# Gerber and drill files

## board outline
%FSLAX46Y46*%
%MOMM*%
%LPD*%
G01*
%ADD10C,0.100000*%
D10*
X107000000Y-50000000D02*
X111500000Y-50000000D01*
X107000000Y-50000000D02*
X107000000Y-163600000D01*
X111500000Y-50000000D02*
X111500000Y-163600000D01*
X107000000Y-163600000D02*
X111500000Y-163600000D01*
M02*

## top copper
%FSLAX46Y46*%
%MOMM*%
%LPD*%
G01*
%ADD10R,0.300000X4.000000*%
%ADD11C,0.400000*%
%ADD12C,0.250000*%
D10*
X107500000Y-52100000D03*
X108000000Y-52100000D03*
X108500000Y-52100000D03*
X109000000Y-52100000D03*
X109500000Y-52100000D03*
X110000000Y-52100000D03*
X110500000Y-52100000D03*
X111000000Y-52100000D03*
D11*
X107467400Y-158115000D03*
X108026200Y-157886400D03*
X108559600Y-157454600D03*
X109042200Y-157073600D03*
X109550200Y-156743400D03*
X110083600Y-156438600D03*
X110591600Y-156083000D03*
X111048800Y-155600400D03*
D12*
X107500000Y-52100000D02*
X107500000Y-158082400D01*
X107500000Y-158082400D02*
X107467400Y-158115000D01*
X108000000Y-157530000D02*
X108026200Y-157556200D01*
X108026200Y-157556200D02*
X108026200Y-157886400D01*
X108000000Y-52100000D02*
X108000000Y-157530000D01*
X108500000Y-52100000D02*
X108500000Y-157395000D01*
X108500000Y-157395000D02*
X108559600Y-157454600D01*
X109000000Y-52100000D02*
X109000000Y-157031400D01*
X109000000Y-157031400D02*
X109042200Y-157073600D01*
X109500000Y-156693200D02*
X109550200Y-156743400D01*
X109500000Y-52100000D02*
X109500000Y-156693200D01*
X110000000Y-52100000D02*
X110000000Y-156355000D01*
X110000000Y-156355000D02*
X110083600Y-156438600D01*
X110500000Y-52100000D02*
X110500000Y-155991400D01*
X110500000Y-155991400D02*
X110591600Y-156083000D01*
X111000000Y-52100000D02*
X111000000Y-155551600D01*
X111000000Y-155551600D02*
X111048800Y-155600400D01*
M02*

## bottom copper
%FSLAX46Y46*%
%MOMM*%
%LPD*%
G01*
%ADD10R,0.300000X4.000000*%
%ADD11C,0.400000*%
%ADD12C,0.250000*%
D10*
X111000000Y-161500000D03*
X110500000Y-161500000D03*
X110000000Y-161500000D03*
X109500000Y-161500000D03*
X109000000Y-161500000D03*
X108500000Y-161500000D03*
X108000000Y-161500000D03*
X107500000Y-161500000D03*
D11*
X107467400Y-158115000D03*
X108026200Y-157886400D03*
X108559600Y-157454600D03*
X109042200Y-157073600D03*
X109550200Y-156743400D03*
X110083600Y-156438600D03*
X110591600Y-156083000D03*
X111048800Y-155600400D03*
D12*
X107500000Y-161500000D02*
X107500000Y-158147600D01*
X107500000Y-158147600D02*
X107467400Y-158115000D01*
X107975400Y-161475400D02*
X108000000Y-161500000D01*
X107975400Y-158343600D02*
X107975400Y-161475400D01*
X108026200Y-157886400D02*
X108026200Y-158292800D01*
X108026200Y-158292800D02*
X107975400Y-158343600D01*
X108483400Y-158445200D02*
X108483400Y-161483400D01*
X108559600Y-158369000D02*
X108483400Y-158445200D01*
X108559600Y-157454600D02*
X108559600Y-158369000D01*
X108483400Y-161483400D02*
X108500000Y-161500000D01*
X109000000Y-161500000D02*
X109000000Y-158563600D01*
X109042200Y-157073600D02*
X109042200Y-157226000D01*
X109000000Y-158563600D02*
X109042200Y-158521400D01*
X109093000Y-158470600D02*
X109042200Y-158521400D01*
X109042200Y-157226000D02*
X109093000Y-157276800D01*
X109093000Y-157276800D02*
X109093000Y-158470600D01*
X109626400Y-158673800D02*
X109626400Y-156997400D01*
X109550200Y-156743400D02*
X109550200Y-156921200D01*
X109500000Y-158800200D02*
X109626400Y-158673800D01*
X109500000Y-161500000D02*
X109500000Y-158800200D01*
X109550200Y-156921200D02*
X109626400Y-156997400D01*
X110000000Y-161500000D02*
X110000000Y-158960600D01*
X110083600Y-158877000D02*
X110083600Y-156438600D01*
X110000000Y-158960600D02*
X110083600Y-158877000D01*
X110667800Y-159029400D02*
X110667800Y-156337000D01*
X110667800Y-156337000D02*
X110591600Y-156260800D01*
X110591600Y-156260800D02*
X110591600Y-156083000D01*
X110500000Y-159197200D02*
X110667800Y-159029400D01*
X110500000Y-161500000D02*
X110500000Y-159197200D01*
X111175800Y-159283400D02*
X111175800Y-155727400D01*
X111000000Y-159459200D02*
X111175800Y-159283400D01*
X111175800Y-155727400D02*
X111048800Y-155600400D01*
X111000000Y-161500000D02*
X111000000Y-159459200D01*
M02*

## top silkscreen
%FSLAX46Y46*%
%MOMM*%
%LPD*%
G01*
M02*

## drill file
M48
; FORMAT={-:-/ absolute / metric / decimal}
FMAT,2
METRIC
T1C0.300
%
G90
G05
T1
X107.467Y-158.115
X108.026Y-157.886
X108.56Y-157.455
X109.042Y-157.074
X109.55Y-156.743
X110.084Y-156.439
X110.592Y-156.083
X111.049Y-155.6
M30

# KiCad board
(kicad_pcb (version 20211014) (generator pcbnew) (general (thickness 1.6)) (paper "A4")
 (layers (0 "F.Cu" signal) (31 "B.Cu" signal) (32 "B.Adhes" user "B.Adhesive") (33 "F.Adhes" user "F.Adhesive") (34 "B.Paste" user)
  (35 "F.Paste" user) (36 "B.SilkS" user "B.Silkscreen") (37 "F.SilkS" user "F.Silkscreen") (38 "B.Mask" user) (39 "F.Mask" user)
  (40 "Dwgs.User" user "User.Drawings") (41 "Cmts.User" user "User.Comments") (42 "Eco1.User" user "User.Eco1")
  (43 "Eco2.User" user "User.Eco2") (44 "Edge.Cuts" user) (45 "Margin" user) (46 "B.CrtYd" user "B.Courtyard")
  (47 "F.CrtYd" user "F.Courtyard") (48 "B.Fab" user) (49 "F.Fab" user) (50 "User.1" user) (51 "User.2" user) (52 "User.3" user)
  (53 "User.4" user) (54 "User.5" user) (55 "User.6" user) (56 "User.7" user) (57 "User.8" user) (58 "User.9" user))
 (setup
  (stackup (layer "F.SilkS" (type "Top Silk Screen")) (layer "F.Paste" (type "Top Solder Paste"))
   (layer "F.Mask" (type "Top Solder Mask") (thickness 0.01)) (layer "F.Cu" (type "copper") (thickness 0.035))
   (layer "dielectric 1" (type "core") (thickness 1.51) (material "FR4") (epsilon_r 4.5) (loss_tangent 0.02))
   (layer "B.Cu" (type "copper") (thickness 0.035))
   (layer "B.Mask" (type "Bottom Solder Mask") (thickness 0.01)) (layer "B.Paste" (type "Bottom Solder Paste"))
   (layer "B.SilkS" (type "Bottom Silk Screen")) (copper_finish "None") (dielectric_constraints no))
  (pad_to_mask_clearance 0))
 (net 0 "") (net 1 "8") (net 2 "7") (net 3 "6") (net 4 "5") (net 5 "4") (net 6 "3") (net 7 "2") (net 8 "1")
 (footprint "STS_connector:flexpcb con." (layer "F.Cu") (at 107 54.1)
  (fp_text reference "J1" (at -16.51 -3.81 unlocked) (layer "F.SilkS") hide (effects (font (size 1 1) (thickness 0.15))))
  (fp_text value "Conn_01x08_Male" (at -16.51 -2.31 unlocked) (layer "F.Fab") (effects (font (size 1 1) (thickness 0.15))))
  (pad "1" smd rect (at 0.5 -2) (size 0.3 4) (layers "F.Cu" "F.Paste" "F.Mask") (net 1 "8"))
  (pad "2" smd rect (at 1 -2) (size 0.3 4) (layers "F.Cu" "F.Paste" "F.Mask") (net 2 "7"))
  (pad "3" smd rect (at 1.5 -2) (size 0.3 4) (layers "F.Cu" "F.Paste" "F.Mask") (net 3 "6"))
  (pad "4" smd rect (at 2 -2) (size 0.3 4) (layers "F.Cu" "F.Paste" "F.Mask") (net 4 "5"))
  (pad "5" smd rect (at 2.5 -2) (size 0.3 4) (layers "F.Cu" "F.Paste" "F.Mask") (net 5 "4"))
  (pad "6" smd rect (at 3 -2) (size 0.3 4) (layers "F.Cu" "F.Paste" "F.Mask") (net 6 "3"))
  (pad "7" smd rect (at 3.5 -2) (size 0.3 4) (layers "F.Cu" "F.Paste" "F.Mask") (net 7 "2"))
  (pad "8" smd rect (at 4 -2) (size 0.3 4) (layers "F.Cu" "F.Paste" "F.Mask") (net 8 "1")))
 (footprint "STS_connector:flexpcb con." (layer "B.Cu") (at 111.5 163.5 180)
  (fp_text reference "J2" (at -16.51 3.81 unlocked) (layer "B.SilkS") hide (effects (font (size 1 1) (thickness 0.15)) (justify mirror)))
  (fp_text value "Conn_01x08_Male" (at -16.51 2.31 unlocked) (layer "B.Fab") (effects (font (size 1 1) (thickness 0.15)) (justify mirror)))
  (pad "1" smd rect (at 0.5 2 180) (size 0.3 4) (layers "B.Cu" "B.Paste" "B.Mask") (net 8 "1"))
  (pad "2" smd rect (at 1 2 180) (size 0.3 4) (layers "B.Cu" "B.Paste" "B.Mask") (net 7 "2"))
  (pad "3" smd rect (at 1.5 2 180) (size 0.3 4) (layers "B.Cu" "B.Paste" "B.Mask") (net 6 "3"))
  (pad "4" smd rect (at 2 2 180) (size 0.3 4) (layers "B.Cu" "B.Paste" "B.Mask") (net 5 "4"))
  (pad "5" smd rect (at 2.5 2 180) (size 0.3 4) (layers "B.Cu" "B.Paste" "B.Mask") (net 4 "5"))
  (pad "6" smd rect (at 3 2 180) (size 0.3 4) (layers "B.Cu" "B.Paste" "B.Mask") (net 3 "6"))
  (pad "7" smd rect (at 3.5 2 180) (size 0.3 4) (layers "B.Cu" "B.Paste" "B.Mask") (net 2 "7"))
  (pad "8" smd rect (at 4 2 180) (size 0.3 4) (layers "B.Cu" "B.Paste" "B.Mask") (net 1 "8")))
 (gr_line (start 107 50) (end 111.5 50) (layer "Edge.Cuts") (width 0.1))
 (gr_line (start 107 50) (end 107 163.6) (layer "Edge.Cuts") (width 0.1))
 (gr_line (start 111.5 50) (end 111.5 163.6) (layer "Edge.Cuts") (width 0.1))
 (gr_line (start 107 163.6) (end 111.5 163.6) (layer "Edge.Cuts") (width 0.1))
 (segment (start 107.5 52.1) (end 107.5 158.0824) (width 0.25) (layer "F.Cu") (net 1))
 (segment (start 107.5 158.0824) (end 107.4674 158.115) (width 0.25) (layer "F.Cu") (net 1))
 (via (at 107.4674 158.115) (size 0.4) (drill 0.3) (layers "F.Cu" "B.Cu") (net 1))
 (segment (start 107.5 161.5) (end 107.5 158.1476) (width 0.25) (layer "B.Cu") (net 1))
 (segment (start 107.5 158.1476) (end 107.4674 158.115) (width 0.25) (layer "B.Cu") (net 1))
 (segment (start 108 157.53) (end 108.0262 157.5562) (width 0.25) (layer "F.Cu") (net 2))
 (segment (start 108.0262 157.5562) (end 108.0262 157.8864) (width 0.25) (layer "F.Cu") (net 2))
 (segment (start 108 52.1) (end 108 157.53) (width 0.25) (layer "F.Cu") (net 2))
 (via (at 108.0262 157.8864) (size 0.4) (drill 0.3) (layers "F.Cu" "B.Cu") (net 2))
 (segment (start 107.9754 161.4754) (end 108 161.5) (width 0.25) (layer "B.Cu") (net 2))
 (segment (start 107.9754 158.3436) (end 107.9754 161.4754) (width 0.25) (layer "B.Cu") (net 2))
 (segment (start 108.0262 157.8864) (end 108.0262 158.2928) (width 0.25) (layer "B.Cu") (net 2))
 (segment (start 108.0262 158.2928) (end 107.9754 158.3436) (width 0.25) (layer "B.Cu") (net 2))
 (segment (start 108.5 52.1) (end 108.5 157.395) (width 0.25) (layer "F.Cu") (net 3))
 (segment (start 108.5 157.395) (end 108.5596 157.4546) (width 0.25) (layer "F.Cu") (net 3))
 (via (at 108.5596 157.4546) (size 0.4) (drill 0.3) (layers "F.Cu" "B.Cu") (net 3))
 (segment (start 108.4834 158.4452) (end 108.4834 161.4834) (width 0.25) (layer "B.Cu") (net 3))
 (segment (start 108.5596 158.369) (end 108.4834 158.4452) (width 0.25) (layer "B.Cu") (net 3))
 (segment (start 108.5596 157.4546) (end 108.5596 158.369) (width 0.25) (layer "B.Cu") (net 3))
 (segment (start 108.4834 161.4834) (end 108.5 161.5) (width 0.25) (layer "B.Cu") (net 3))
 (segment (start 109 52.1) (end 109 157.0314) (width 0.25) (layer "F.Cu") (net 4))
 (segment (start 109 157.0314) (end 109.0422 157.0736) (width 0.25) (layer "F.Cu") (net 4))
 (via (at 109.0422 157.0736) (size 0.4) (drill 0.3) (layers "F.Cu" "B.Cu") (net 4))
 (segment (start 109 161.5) (end 109 158.5636) (width 0.25) (layer "B.Cu") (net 4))
 (segment (start 109.0422 157.0736) (end 109.0422 157.226) (width 0.25) (layer "B.Cu") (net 4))
 (segment (start 109 158.5636) (end 109.0422 158.5214) (width 0.25) (layer "B.Cu") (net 4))
 (segment (start 109.093 158.4706) (end 109.0422 158.5214) (width 0.25) (layer "B.Cu") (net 4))
 (segment (start 109.0422 157.226) (end 109.093 157.2768) (width 0.25) (layer "B.Cu") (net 4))
 (segment (start 109.093 157.2768) (end 109.093 158.4706) (width 0.25) (layer "B.Cu") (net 4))
 (segment (start 109.5 156.6932) (end 109.5502 156.7434) (width 0.25) (layer "F.Cu") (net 5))
 (segment (start 109.5 52.1) (end 109.5 156.6932) (width 0.25) (layer "F.Cu") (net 5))
 (via (at 109.5502 156.7434) (size 0.4) (drill 0.3) (layers "F.Cu" "B.Cu") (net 5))
 (segment (start 109.6264 158.6738) (end 109.6264 156.9974) (width 0.25) (layer "B.Cu") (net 5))
 (segment (start 109.5502 156.7434) (end 109.5502 156.9212) (width 0.25) (layer "B.Cu") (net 5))
 (segment (start 109.5 158.8002) (end 109.6264 158.6738) (width 0.25) (layer "B.Cu") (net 5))
 (segment (start 109.5 161.5) (end 109.5 158.8002) (width 0.25) (layer "B.Cu") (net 5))
 (segment (start 109.5502 156.9212) (end 109.6264 156.9974) (width 0.25) (layer "B.Cu") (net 5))
 (segment (start 110 52.1) (end 110 156.355) (width 0.25) (layer "F.Cu") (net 6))
 (segment (start 110 156.355) (end 110.0836 156.4386) (width 0.25) (layer "F.Cu") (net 6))
 (via (at 110.0836 156.4386) (size 0.4) (drill 0.3) (layers "F.Cu" "B.Cu") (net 6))
 (segment (start 110 161.5) (end 110 158.9606) (width 0.25) (layer "B.Cu") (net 6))
 (segment (start 110.0836 158.877) (end 110.0836 156.4386) (width 0.25) (layer "B.Cu") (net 6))
 (segment (start 110 158.9606) (end 110.0836 158.877) (width 0.25) (layer "B.Cu") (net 6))
 (segment (start 110.5 52.1) (end 110.5 155.9914) (width 0.25) (layer "F.Cu") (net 7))
 (segment (start 110.5 155.9914) (end 110.5916 156.083) (width 0.25) (layer "F.Cu") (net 7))
 (via (at 110.5916 156.083) (size 0.4) (drill 0.3) (layers "F.Cu" "B.Cu") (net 7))
 (segment (start 110.6678 159.0294) (end 110.6678 156.337) (width 0.25) (layer "B.Cu") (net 7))
 (segment (start 110.6678 156.337) (end 110.5916 156.2608) (width 0.25) (layer "B.Cu") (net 7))
 (segment (start 110.5916 156.2608) (end 110.5916 156.083) (width 0.25) (layer "B.Cu") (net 7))
 (segment (start 110.5 159.1972) (end 110.6678 159.0294) (width 0.25) (layer "B.Cu") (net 7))
 (segment (start 110.5 161.5) (end 110.5 159.1972) (width 0.25) (layer "B.Cu") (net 7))
 (segment (start 111 52.1) (end 111 155.5516) (width 0.25) (layer "F.Cu") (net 8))
 (segment (start 111 155.5516) (end 111.0488 155.6004) (width 0.25) (layer "F.Cu") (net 8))
 (via (at 111.0488 155.6004) (size 0.4) (drill 0.3) (layers "F.Cu" "B.Cu") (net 8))
 (segment (start 111.1758 159.2834) (end 111.1758 155.7274) (width 0.25) (layer "B.Cu") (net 8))
 (segment (start 111 159.4592) (end 111.1758 159.2834) (width 0.25) (layer "B.Cu") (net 8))
 (segment (start 111.1758 155.7274) (end 111.0488 155.6004) (width 0.25) (layer "B.Cu") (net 8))
 (segment (start 111 161.5) (end 111 159.4592) (width 0.25) (layer "B.Cu") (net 8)))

